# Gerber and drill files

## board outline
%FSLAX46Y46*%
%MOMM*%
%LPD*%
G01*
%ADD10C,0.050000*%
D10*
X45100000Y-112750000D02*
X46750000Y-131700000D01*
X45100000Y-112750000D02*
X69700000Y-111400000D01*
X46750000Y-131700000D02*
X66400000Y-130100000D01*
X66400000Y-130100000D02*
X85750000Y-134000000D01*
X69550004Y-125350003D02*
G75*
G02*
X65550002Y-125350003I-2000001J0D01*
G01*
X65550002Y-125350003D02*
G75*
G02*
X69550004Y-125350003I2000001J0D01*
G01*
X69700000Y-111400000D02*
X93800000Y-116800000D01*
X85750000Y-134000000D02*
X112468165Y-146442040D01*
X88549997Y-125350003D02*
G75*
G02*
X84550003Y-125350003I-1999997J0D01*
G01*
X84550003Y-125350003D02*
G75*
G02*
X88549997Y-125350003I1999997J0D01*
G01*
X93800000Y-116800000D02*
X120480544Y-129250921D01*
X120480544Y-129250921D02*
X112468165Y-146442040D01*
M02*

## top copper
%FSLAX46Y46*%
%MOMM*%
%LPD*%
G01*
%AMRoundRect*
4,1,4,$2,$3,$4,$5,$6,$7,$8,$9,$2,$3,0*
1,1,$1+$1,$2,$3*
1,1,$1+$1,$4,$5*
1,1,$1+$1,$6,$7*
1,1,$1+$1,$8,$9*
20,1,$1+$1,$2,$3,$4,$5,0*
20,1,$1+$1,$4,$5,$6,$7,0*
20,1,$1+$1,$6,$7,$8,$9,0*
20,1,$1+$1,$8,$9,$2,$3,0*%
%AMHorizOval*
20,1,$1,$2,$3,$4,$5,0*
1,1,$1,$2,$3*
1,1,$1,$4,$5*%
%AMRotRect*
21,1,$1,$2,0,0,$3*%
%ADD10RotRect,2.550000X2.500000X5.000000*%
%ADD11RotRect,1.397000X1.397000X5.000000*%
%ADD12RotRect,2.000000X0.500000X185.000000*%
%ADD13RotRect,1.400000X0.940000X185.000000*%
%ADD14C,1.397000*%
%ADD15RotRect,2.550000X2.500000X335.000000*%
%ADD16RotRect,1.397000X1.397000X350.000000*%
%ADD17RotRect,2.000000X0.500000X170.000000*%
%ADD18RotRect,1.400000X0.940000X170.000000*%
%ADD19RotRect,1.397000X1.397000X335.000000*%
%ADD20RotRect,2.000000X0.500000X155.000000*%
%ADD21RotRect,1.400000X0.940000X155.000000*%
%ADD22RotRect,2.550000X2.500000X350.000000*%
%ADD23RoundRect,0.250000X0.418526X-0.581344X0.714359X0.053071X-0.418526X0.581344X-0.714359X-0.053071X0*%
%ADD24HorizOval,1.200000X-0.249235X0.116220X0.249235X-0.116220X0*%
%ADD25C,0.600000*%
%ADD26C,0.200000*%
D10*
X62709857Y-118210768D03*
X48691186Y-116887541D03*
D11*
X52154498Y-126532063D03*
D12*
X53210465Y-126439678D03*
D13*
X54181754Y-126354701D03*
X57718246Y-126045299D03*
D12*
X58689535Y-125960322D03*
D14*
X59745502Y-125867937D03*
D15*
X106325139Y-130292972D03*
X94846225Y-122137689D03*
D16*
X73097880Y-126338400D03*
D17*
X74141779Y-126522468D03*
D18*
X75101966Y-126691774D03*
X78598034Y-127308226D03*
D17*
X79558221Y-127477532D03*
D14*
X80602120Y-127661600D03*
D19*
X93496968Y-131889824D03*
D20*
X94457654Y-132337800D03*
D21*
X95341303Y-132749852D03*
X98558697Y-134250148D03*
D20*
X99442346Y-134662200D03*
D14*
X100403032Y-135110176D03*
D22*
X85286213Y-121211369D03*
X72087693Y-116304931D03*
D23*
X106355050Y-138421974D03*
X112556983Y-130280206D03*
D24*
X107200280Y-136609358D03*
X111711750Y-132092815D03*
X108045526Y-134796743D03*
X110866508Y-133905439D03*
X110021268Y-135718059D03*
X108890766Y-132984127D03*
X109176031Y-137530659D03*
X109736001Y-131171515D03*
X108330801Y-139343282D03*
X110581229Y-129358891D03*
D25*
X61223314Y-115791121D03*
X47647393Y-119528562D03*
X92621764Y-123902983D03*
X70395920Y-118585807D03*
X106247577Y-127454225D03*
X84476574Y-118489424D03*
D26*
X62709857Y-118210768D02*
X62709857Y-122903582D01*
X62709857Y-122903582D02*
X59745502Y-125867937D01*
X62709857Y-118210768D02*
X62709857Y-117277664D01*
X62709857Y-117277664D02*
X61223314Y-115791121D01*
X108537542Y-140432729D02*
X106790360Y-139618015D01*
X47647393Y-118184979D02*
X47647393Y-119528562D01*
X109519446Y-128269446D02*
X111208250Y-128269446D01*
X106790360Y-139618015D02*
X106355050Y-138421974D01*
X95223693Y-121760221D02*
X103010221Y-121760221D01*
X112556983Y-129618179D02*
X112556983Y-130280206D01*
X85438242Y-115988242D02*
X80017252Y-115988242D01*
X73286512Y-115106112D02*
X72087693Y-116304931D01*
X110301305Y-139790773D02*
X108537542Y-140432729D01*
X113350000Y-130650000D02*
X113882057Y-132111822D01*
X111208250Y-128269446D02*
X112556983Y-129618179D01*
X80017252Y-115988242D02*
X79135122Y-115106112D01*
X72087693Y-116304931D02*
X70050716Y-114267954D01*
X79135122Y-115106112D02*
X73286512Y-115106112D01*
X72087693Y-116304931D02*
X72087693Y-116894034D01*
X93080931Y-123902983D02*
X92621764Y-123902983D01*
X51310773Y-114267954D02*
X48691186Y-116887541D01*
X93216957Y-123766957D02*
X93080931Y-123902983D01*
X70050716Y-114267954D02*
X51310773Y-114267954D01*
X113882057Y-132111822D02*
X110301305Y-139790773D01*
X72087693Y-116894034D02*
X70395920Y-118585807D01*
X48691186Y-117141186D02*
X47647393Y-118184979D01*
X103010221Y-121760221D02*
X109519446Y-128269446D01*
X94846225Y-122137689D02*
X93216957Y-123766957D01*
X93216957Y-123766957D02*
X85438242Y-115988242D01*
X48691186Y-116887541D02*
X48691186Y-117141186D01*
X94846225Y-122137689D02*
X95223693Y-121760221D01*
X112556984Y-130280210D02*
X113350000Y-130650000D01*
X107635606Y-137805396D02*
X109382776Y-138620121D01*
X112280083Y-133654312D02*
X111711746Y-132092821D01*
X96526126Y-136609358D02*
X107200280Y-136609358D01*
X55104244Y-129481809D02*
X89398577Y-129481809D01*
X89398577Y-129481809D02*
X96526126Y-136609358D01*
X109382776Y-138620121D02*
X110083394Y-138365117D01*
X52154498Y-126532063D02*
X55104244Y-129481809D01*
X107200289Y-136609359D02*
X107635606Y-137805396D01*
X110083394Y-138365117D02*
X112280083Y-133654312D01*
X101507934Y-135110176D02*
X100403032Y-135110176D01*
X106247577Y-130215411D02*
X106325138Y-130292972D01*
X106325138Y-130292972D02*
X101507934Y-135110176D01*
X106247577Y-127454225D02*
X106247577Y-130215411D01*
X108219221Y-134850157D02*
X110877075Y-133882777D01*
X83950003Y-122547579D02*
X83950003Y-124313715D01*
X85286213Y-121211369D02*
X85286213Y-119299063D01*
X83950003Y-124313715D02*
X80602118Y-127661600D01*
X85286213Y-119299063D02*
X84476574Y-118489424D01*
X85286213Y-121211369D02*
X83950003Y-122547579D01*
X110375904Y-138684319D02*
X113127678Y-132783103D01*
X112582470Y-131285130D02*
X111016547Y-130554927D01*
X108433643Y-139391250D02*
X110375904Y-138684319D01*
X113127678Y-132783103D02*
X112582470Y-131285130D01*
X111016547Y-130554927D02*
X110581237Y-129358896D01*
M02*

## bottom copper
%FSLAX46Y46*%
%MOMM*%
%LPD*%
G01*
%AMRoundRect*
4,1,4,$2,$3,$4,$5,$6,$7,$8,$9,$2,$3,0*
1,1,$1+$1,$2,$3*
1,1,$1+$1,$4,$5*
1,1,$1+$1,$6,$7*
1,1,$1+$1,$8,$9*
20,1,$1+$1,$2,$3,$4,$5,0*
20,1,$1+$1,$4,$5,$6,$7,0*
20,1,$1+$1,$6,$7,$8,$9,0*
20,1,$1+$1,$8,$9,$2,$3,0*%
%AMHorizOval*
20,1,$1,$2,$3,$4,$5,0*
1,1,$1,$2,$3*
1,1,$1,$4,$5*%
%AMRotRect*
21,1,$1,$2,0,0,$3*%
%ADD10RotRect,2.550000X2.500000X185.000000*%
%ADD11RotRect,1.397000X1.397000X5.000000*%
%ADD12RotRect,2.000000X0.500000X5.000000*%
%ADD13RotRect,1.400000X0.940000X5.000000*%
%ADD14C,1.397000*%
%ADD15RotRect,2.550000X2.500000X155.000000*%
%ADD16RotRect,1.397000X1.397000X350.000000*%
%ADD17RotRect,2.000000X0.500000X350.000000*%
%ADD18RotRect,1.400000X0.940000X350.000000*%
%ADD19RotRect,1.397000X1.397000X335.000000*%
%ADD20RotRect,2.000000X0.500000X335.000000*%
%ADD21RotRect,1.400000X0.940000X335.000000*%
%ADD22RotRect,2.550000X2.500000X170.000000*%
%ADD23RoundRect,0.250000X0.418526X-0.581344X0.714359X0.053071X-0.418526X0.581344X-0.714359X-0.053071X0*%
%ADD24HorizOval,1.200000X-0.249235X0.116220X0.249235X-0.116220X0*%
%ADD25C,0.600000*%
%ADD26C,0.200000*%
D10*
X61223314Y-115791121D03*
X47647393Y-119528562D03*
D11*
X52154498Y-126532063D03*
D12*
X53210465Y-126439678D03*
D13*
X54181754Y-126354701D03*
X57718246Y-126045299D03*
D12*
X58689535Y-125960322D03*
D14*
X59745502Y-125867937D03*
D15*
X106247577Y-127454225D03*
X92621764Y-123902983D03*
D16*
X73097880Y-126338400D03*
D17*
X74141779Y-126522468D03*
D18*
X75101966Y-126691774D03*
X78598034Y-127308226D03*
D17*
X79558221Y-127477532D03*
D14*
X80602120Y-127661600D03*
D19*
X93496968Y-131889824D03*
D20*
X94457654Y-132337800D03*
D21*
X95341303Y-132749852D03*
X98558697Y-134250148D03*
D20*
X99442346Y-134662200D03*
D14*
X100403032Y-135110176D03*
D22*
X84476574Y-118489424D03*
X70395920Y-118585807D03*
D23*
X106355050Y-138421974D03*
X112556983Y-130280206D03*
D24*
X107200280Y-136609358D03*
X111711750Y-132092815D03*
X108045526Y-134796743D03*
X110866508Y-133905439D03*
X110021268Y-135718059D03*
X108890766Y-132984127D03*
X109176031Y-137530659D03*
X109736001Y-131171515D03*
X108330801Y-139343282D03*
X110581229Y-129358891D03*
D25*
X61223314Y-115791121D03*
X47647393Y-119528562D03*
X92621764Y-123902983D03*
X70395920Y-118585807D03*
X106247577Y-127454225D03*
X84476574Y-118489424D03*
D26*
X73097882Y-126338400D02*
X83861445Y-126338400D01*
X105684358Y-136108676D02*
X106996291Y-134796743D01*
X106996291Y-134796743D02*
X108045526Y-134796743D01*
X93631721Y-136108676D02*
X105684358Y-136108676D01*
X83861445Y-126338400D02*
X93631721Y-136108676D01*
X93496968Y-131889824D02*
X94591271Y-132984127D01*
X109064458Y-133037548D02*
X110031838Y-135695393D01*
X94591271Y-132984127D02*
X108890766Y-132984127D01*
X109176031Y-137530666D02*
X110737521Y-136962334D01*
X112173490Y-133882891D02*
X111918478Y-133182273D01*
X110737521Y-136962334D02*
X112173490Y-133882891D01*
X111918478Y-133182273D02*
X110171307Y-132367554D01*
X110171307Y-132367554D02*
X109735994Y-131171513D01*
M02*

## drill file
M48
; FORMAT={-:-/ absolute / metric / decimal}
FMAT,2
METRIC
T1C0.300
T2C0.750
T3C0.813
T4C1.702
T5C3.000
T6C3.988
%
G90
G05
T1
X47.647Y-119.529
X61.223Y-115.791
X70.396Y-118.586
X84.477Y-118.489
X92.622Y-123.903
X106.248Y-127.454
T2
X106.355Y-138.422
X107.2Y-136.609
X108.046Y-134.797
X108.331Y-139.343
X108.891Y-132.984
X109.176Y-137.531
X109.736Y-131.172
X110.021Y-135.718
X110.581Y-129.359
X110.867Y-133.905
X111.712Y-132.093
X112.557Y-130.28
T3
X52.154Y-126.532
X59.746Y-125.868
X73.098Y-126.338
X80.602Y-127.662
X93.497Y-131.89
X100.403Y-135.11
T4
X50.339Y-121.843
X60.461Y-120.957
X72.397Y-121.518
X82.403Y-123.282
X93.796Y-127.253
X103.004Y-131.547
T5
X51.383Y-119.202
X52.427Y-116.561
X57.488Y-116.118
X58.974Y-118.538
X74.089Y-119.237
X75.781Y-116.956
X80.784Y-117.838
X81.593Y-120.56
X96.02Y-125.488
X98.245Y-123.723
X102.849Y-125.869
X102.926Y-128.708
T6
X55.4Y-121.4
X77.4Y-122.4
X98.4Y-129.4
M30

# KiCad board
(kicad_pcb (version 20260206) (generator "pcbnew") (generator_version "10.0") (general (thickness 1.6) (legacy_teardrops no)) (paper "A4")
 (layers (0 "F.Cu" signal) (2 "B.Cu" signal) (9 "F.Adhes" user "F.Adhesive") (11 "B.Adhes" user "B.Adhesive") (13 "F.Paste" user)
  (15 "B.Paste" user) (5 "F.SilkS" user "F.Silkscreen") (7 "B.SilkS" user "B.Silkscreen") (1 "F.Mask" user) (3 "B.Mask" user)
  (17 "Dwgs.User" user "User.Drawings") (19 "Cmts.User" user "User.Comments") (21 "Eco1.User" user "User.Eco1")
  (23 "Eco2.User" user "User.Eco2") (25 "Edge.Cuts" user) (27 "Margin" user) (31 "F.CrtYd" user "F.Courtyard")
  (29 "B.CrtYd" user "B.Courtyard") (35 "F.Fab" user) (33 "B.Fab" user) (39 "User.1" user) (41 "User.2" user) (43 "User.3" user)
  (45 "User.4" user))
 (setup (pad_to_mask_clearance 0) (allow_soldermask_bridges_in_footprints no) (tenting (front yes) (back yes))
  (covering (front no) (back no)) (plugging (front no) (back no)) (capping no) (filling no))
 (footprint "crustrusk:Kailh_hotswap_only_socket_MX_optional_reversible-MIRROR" (layer "F.Cu") (at 55.400001 121.4 5)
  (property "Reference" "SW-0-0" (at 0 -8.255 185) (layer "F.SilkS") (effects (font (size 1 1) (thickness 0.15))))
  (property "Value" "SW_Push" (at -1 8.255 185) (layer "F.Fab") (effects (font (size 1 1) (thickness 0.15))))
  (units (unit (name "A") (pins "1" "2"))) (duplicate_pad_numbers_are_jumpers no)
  (pad "" np_thru_hole circle (at -5.08 0 5) (size 1.7018 1.7018) (drill 1.7018) (layers "*.Cu" "*.Mask"))
  (pad "" np_thru_hole circle (at -3.81 -2.54 185) (size 3 3) (drill 3) (layers "*.Cu" "*.Mask"))
  (pad "" np_thru_hole circle (at -2.540002 -5.079998 5) (size 3 3) (drill 3) (layers "*.Cu" "*.Mask"))
  (pad "" np_thru_hole circle (at 0 0 5) (size 3.9878 3.9878) (drill 3.9878) (layers "*.Cu" "*.Mask"))
  (pad "" np_thru_hole circle (at 2.540002 -5.080001 185) (size 3 3) (drill 3) (layers "*.Cu" "*.Mask"))
  (pad "" np_thru_hole circle (at 3.81 -2.54 5) (size 3 3) (drill 3) (layers "*.Cu" "*.Mask"))
  (pad "" np_thru_hole circle (at 5.08 0 5) (size 1.7018 1.7018) (drill 1.7018) (layers "*.Cu" "*.Mask"))
  (pad "1" smd rect (at 6.29 -5.08 185) (size 2.55 2.5) (layers "B.Cu" "B.Mask" "B.Paste") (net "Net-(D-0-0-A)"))
  (pad "1" smd rect (at 7.56 -2.54 5) (size 2.55 2.5) (layers "F.Cu" "F.Mask" "F.Paste") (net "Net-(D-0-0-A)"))
  (pad "2" smd rect (at -7.56 -2.540001 185) (size 2.55 2.5) (layers "B.Cu" "B.Mask" "B.Paste") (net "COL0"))
  (pad "2" smd rect (at -6.289999 -5.079999 5) (size 2.55 2.5) (layers "F.Cu" "F.Mask" "F.Paste") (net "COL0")))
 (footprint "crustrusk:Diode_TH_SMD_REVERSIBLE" (layer "F.Cu") (at 55.95 126.2 5)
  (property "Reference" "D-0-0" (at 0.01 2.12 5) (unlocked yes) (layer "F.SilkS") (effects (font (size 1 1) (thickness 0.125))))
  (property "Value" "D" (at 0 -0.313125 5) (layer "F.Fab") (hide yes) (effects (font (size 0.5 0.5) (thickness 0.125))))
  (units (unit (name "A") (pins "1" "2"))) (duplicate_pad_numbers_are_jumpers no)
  (pad "1" thru_hole rect (at -3.81 0 5) (size 1.397 1.397) (drill 0.8128) (layers "*.Cu" "*.Mask") (remove_unused_layers no) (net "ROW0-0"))
  (pad "1" smd rect (at -2.75 0 185) (size 2 0.5) (layers "F.Cu") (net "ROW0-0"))
  (pad "1" smd rect (at -2.75 0 5) (size 2 0.5) (layers "B.Cu") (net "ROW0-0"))
  (pad "1" smd rect (at -1.775 0 185) (size 1.4 0.94) (layers "F.Cu" "F.Mask" "F.Paste") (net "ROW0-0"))
  (pad "1" smd rect (at -1.775 0 5) (size 1.4 0.94) (layers "B.Cu" "B.Mask" "B.Paste") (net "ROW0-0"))
  (pad "2" smd rect (at 1.775 0 185) (size 1.4 0.94) (layers "F.Cu" "F.Mask" "F.Paste") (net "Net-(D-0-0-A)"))
  (pad "2" smd rect (at 1.775 0 5) (size 1.4 0.94) (layers "B.Cu" "B.Mask" "B.Paste") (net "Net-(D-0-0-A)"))
  (pad "2" smd rect (at 2.75 0 185) (size 2 0.5) (layers "F.Cu") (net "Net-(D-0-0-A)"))
  (pad "2" smd rect (at 2.75 0 5) (size 2 0.5) (layers "B.Cu") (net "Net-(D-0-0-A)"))
  (pad "2" thru_hole circle (at 3.81 0 5) (size 1.397 1.397) (drill 0.8128) (layers "*.Cu" "*.Mask") (remove_unused_layers no)
   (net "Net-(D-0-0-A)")))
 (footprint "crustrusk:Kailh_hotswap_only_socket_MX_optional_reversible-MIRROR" (layer "F.Cu") (at 98.4 129.4 -25)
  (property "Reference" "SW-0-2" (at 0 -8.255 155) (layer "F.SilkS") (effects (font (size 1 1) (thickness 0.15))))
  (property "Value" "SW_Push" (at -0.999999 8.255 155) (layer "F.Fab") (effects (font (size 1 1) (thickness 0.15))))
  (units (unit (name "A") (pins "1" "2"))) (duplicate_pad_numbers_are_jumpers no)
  (pad "" np_thru_hole circle (at -5.08 0 335) (size 1.7018 1.7018) (drill 1.7018) (layers "*.Cu" "*.Mask"))
  (pad "" np_thru_hole circle (at -3.81 -2.539998 155) (size 3 3) (drill 3) (layers "*.Cu" "*.Mask"))
  (pad "" np_thru_hole circle (at -2.54 -5.079998 335) (size 3 3) (drill 3) (layers "*.Cu" "*.Mask"))
  (pad "" np_thru_hole circle (at 0 0 335) (size 3.9878 3.9878) (drill 3.9878) (layers "*.Cu" "*.Mask"))
  (pad "" np_thru_hole circle (at 2.540002 -5.080001 155) (size 3 3) (drill 3) (layers "*.Cu" "*.Mask"))
  (pad "" np_thru_hole circle (at 3.81 -2.54 335) (size 3 3) (drill 3) (layers "*.Cu" "*.Mask"))
  (pad "" np_thru_hole circle (at 5.08 0 335) (size 1.7018 1.7018) (drill 1.7018) (layers "*.Cu" "*.Mask"))
  (pad "1" smd rect (at 6.29 -5.08 155) (size 2.55 2.5) (layers "B.Cu" "B.Mask" "B.Paste") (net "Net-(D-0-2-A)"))
  (pad "1" smd rect (at 7.560001 -2.540001 335) (size 2.55 2.5) (layers "F.Cu" "F.Mask" "F.Paste") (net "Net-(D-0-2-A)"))
  (pad "2" smd rect (at -7.56 -2.540001 155) (size 2.55 2.5) (layers "B.Cu" "B.Mask" "B.Paste") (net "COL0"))
  (pad "2" smd rect (at -6.289999 -5.079999 335) (size 2.55 2.5) (layers "F.Cu" "F.Mask" "F.Paste") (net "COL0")))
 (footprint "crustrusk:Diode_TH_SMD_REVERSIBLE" (layer "F.Cu") (at 76.85 127 -10)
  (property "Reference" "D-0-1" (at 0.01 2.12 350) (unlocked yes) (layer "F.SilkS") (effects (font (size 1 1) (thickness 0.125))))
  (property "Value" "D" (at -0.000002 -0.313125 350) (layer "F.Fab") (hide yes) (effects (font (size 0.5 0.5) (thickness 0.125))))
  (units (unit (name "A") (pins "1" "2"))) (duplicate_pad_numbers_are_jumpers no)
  (pad "1" thru_hole rect (at -3.810002 0 350) (size 1.397 1.397) (drill 0.8128) (layers "*.Cu" "*.Mask") (remove_unused_layers no)
   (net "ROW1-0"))
  (pad "1" smd rect (at -2.75 0 170) (size 2 0.5) (layers "F.Cu") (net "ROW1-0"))
  (pad "1" smd rect (at -2.75 0 350) (size 2 0.5) (layers "B.Cu") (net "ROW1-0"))
  (pad "1" smd rect (at -1.775 0 170) (size 1.4 0.94) (layers "F.Cu" "F.Mask" "F.Paste") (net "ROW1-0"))
  (pad "1" smd rect (at -1.775 0 350) (size 1.4 0.94) (layers "B.Cu" "B.Mask" "B.Paste") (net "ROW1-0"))
  (pad "2" smd rect (at 1.775 0 170) (size 1.4 0.94) (layers "F.Cu" "F.Mask" "F.Paste") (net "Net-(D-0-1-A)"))
  (pad "2" smd rect (at 1.775 0 350) (size 1.4 0.94) (layers "B.Cu" "B.Mask" "B.Paste") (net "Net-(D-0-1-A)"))
  (pad "2" smd rect (at 2.75 0 170) (size 2 0.5) (layers "F.Cu") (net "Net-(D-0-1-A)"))
  (pad "2" smd rect (at 2.75 0 350) (size 2 0.5) (layers "B.Cu") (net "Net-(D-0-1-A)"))
  (pad "2" thru_hole circle (at 3.810002 0 350) (size 1.397 1.397) (drill 0.8128) (layers "*.Cu" "*.Mask") (remove_unused_layers no)
   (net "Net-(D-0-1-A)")))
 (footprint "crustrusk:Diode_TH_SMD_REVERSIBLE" (layer "F.Cu") (at 96.95 133.5 -25)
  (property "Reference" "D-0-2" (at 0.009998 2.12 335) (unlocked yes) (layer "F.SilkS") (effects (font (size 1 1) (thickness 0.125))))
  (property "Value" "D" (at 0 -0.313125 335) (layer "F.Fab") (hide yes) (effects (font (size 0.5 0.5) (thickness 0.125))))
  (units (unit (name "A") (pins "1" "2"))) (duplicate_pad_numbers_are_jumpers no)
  (pad "1" thru_hole rect (at -3.81 -0.000001 335) (size 1.397 1.397) (drill 0.8128) (layers "*.Cu" "*.Mask") (remove_unused_layers no)
   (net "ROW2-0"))
  (pad "1" smd rect (at -2.75 0 155) (size 2 0.5) (layers "F.Cu") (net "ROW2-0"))
  (pad "1" smd rect (at -2.75 0 335) (size 2 0.5) (layers "B.Cu") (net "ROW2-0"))
  (pad "1" smd rect (at -1.775001 0 155) (size 1.4 0.94) (layers "F.Cu" "F.Mask" "F.Paste") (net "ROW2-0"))
  (pad "1" smd rect (at -1.775001 0 335) (size 1.4 0.94) (layers "B.Cu" "B.Mask" "B.Paste") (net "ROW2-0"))
  (pad "2" smd rect (at 1.775001 0 155) (size 1.4 0.94) (layers "F.Cu" "F.Mask" "F.Paste") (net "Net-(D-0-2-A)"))
  (pad "2" smd rect (at 1.775001 0 335) (size 1.4 0.94) (layers "B.Cu" "B.Mask" "B.Paste") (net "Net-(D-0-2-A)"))
  (pad "2" smd rect (at 2.75 0 155) (size 2 0.5) (layers "F.Cu") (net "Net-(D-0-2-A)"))
  (pad "2" smd rect (at 2.75 0 335) (size 2 0.5) (layers "B.Cu") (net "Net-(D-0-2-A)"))
  (pad "2" thru_hole circle (at 3.81 0.000001 335) (size 1.397 1.397) (drill 0.8128) (layers "*.Cu" "*.Mask") (remove_unused_layers no)
   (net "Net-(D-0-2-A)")))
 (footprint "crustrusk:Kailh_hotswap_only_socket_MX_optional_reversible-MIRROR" (layer "F.Cu") (at 77.4 122.4 -10)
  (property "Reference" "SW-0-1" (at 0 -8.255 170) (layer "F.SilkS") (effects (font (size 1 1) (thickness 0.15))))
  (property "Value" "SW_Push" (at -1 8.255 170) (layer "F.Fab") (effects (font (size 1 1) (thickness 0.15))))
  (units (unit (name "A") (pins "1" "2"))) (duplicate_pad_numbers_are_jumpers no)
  (pad "" np_thru_hole circle (at -5.08 0 350) (size 1.7018 1.7018) (drill 1.7018) (layers "*.Cu" "*.Mask"))
  (pad "" np_thru_hole circle (at -3.81 -2.54 170) (size 3 3) (drill 3) (layers "*.Cu" "*.Mask"))
  (pad "" np_thru_hole circle (at -2.54 -5.079998 350) (size 3 3) (drill 3) (layers "*.Cu" "*.Mask"))
  (pad "" np_thru_hole circle (at 0 0 350) (size 3.9878 3.9878) (drill 3.9878) (layers "*.Cu" "*.Mask"))
  (pad "" np_thru_hole circle (at 2.540002 -5.080001 170) (size 3 3) (drill 3) (layers "*.Cu" "*.Mask"))
  (pad "" np_thru_hole circle (at 3.81 -2.54 350) (size 3 3) (drill 3) (layers "*.Cu" "*.Mask"))
  (pad "" np_thru_hole circle (at 5.08 0 350) (size 1.7018 1.7018) (drill 1.7018) (layers "*.Cu" "*.Mask"))
  (pad "1" smd rect (at 6.290001 -5.08 170) (size 2.55 2.5) (layers "B.Cu" "B.Mask" "B.Paste") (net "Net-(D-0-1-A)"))
  (pad "1" smd rect (at 7.56 -2.54 350) (size 2.55 2.5) (layers "F.Cu" "F.Mask" "F.Paste") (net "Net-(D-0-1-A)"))
  (pad "2" smd rect (at -7.56 -2.540001 170) (size 2.55 2.5) (layers "B.Cu" "B.Mask" "B.Paste") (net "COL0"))
  (pad "2" smd rect (at -6.289999 -5.079999 350) (size 2.55 2.5) (layers "F.Cu" "F.Mask" "F.Paste") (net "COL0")))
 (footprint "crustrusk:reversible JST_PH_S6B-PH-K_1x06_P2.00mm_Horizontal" (layer "F.Cu") (at 106.35505 138.421974 65)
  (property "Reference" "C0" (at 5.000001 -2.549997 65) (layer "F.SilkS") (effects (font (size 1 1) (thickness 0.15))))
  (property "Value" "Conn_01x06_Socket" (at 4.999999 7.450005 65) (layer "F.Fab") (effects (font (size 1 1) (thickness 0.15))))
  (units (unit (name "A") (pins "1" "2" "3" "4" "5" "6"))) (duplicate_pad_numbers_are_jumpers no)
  (pad "1" thru_hole roundrect (at 0 0 65) (size 1.2 1.75) (drill 0.75) (layers "*.Cu" "*.Mask") (remove_unused_layers no)
   (roundrect_rratio 0.208333) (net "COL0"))
  (pad "1" thru_hole roundrect (at 9.999998 2.18 65) (size 1.2 1.75) (drill 0.75) (layers "*.Cu" "*.Mask") (remove_unused_layers no)
   (roundrect_rratio 0.208333) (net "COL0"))
  (pad "2" thru_hole oval (at 1.999998 -0.000006 65) (size 1.2 1.75) (drill 0.75) (layers "*.Cu" "*.Mask") (remove_unused_layers no)
   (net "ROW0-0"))
  (pad "2" thru_hole oval (at 8.000005 2.180001 65) (size 1.2 1.75) (drill 0.75) (layers "*.Cu" "*.Mask") (remove_unused_layers no)
   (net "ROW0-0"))
  (pad "3" thru_hole oval (at 4.000001 0.000003 65) (size 1.2 1.75) (drill 0.75) (layers "*.Cu" "*.Mask") (remove_unused_layers no)
   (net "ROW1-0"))
  (pad "3" thru_hole oval (at 5.999995 2.179999 65) (size 1.2 1.75) (drill 0.75) (layers "*.Cu" "*.Mask") (remove_unused_layers no)
   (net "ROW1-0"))
  (pad "4" thru_hole oval (at 3.99999 2.179998 65) (size 1.2 1.75) (drill 0.75) (layers "*.Cu" "*.Mask") (remove_unused_layers no)
   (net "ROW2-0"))
  (pad "4" thru_hole oval (at 6.000003 0.000006 65) (size 1.2 1.75) (drill 0.75) (layers "*.Cu" "*.Mask") (remove_unused_layers no)
   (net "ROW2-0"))
  (pad "5" thru_hole oval (at 2.000004 2.179991 65) (size 1.2 1.75) (drill 0.75) (layers "*.Cu" "*.Mask") (remove_unused_layers no)
   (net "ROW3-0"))
  (pad "5" thru_hole oval (at 7.999999 0.000006 65) (size 1.2 1.75) (drill 0.75) (layers "*.Cu" "*.Mask") (remove_unused_layers no)
   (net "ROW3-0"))
  (pad "6" thru_hole oval (at 0 2.18 65) (size 1.2 1.75) (drill 0.75) (layers "*.Cu" "*.Mask") (remove_unused_layers no) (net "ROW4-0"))
  (pad "6" thru_hole oval (at 10.000003 -0.000005 65) (size 1.2 1.75) (drill 0.75) (layers "*.Cu" "*.Mask") (remove_unused_layers no)
   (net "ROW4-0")))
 (gr_line (start 45.1 112.75) (end 46.75 131.7) (stroke (width 0.05) (type default)) (layer "Edge.Cuts"))
 (gr_line (start 45.1 112.75) (end 69.7 111.4) (stroke (width 0.05) (type default)) (layer "Edge.Cuts"))
 (gr_line (start 46.75 131.7) (end 66.4 130.1) (stroke (width 0.05) (type default)) (layer "Edge.Cuts"))
 (gr_line (start 66.4 130.1) (end 85.75 134) (stroke (width 0.05) (type default)) (layer "Edge.Cuts"))
 (gr_circle (center 67.550003 125.350003) (end 65.550002 125.350003) (stroke (width 0.05) (type default)) (fill no) (layer "Edge.Cuts"))
 (gr_line (start 69.7 111.4) (end 93.8 116.8) (stroke (width 0.05) (type default)) (layer "Edge.Cuts"))
 (gr_line (start 85.75 134) (end 112.468165 146.44204) (stroke (width 0.05) (type default)) (layer "Edge.Cuts"))
 (gr_circle (center 86.55 125.350003) (end 84.550003 125.350003) (stroke (width 0.05) (type default)) (fill no) (layer "Edge.Cuts"))
 (gr_line (start 93.8 116.8) (end 120.480544 129.250921) (stroke (width 0.05) (type default)) (layer "Edge.Cuts"))
 (gr_line (start 120.480544 129.250921) (end 112.468165 146.44204) (stroke (width 0.05) (type default)) (layer "Edge.Cuts"))
 (segment (start 62.709857 118.210768) (end 62.709857 122.903582) (width 0.2) (layer "F.Cu") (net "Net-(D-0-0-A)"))
 (segment (start 62.709857 122.903582) (end 59.745502 125.867937) (width 0.2) (layer "F.Cu") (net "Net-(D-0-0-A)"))
 (segment (start 62.709857 118.210768) (end 62.709857 117.277664) (width 0.2) (layer "F.Cu") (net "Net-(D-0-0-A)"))
 (segment (start 62.709857 117.277664) (end 61.223314 115.791121) (width 0.2) (layer "F.Cu") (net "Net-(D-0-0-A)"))
 (via (at 61.223314 115.791121) (size 0.6) (drill 0.3) (layers "F.Cu" "B.Cu") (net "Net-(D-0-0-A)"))
 (segment (start 108.537542 140.432729) (end 106.79036 139.618015) (width 0.2) (layer "F.Cu") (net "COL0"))
 (segment (start 47.647393 118.184979) (end 47.647393 119.528562) (width 0.2) (layer "F.Cu") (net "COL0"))
 (segment (start 109.519446 128.269446) (end 111.20825 128.269446) (width 0.2) (layer "F.Cu") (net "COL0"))
 (segment (start 106.79036 139.618015) (end 106.35505 138.421974) (width 0.2) (layer "F.Cu") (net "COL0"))
 (segment (start 95.223693 121.760221) (end 103.010221 121.760221) (width 0.2) (layer "F.Cu") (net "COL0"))
 (segment (start 112.556983 129.618179) (end 112.556983 130.280206) (width 0.2) (layer "F.Cu") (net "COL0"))
 (segment (start 85.438242 115.988242) (end 80.017252 115.988242) (width 0.2) (layer "F.Cu") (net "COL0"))
 (segment (start 73.286512 115.106112) (end 72.087693 116.304931) (width 0.2) (layer "F.Cu") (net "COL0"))
 (segment (start 110.301305 139.790773) (end 108.537542 140.432729) (width 0.2) (layer "F.Cu") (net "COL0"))
 (segment (start 113.35 130.65) (end 113.882057 132.111822) (width 0.2) (layer "F.Cu") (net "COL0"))
 (segment (start 111.20825 128.269446) (end 112.556983 129.618179) (width 0.2) (layer "F.Cu") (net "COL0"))
 (segment (start 80.017252 115.988242) (end 79.135122 115.106112) (width 0.2) (layer "F.Cu") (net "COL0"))
 (segment (start 72.087693 116.304931) (end 70.050716 114.267954) (width 0.2) (layer "F.Cu") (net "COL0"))
 (segment (start 79.135122 115.106112) (end 73.286512 115.106112) (width 0.2) (layer "F.Cu") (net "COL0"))
 (segment (start 72.087693 116.304931) (end 72.087693 116.894034) (width 0.2) (layer "F.Cu") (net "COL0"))
 (segment (start 93.080931 123.902983) (end 92.621764 123.902983) (width 0.2) (layer "F.Cu") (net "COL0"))
 (segment (start 51.310773 114.267954) (end 48.691186 116.887541) (width 0.2) (layer "F.Cu") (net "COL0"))
 (segment (start 93.216957 123.766957) (end 93.080931 123.902983) (width 0.2) (layer "F.Cu") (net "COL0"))
 (segment (start 70.050716 114.267954) (end 51.310773 114.267954) (width 0.2) (layer "F.Cu") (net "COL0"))
 (segment (start 113.882057 132.111822) (end 110.301305 139.790773) (width 0.2) (layer "F.Cu") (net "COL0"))
 (segment (start 72.087693 116.894034) (end 70.39592 118.585807) (width 0.2) (layer "F.Cu") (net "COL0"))
 (segment (start 48.691186 117.141186) (end 47.647393 118.184979) (width 0.2) (layer "F.Cu") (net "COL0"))
 (segment (start 103.010221 121.760221) (end 109.519446 128.269446) (width 0.2) (layer "F.Cu") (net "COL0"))
 (segment (start 94.846225 122.137689) (end 93.216957 123.766957) (width 0.2) (layer "F.Cu") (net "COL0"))
 (segment (start 93.216957 123.766957) (end 85.438242 115.988242) (width 0.2) (layer "F.Cu") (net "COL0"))
 (segment (start 48.691186 116.887541) (end 48.691186 117.141186) (width 0.2) (layer "F.Cu") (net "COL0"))
 (segment (start 94.846225 122.137689) (end 95.223693 121.760221) (width 0.2) (layer "F.Cu") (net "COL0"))
 (segment (start 112.556984 130.28021) (end 113.35 130.65) (width 0.2) (layer "F.Cu") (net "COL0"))
 (via (at 47.647393 119.528562) (size 0.6) (drill 0.3) (layers "F.Cu" "B.Cu") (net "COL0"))
 (via (at 92.621764 123.902983) (size 0.6) (drill 0.3) (layers "F.Cu" "B.Cu") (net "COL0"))
 (via (at 70.39592 118.585807) (size 0.6) (drill 0.3) (layers "F.Cu" "B.Cu") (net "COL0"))
 (segment (start 107.635606 137.805396) (end 109.382776 138.620121) (width 0.2) (layer "F.Cu") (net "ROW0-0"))
 (segment (start 112.280083 133.654312) (end 111.711746 132.092821) (width 0.2) (layer "F.Cu") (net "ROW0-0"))
 (segment (start 96.526126 136.609358) (end 107.20028 136.609358) (width 0.2) (layer "F.Cu") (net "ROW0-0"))
 (segment (start 55.104244 129.481809) (end 89.398577 129.481809) (width 0.2) (layer "F.Cu") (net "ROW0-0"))
 (segment (start 89.398577 129.481809) (end 96.526126 136.609358) (width 0.2) (layer "F.Cu") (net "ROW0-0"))
 (segment (start 109.382776 138.620121) (end 110.083394 138.365117) (width 0.2) (layer "F.Cu") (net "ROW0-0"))
 (segment (start 52.154498 126.532063) (end 55.104244 129.481809) (width 0.2) (layer "F.Cu") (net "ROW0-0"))
 (segment (start 107.200289 136.609359) (end 107.635606 137.805396) (width 0.2) (layer "F.Cu") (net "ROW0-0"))
 (segment (start 110.083394 138.365117) (end 112.280083 133.654312) (width 0.2) (layer "F.Cu") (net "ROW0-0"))
 (segment (start 101.507934 135.110176) (end 100.403032 135.110176) (width 0.2) (layer "F.Cu") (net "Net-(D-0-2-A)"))
 (segment (start 106.247577 130.215411) (end 106.325138 130.292972) (width 0.2) (layer "F.Cu") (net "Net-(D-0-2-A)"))
 (segment (start 106.325138 130.292972) (end 101.507934 135.110176) (width 0.2) (layer "F.Cu") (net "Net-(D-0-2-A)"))
 (segment (start 106.247577 127.454225) (end 106.247577 130.215411) (width 0.2) (layer "F.Cu") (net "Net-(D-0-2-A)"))
 (via (at 106.247577 127.454225) (size 0.6) (drill 0.3) (layers "F.Cu" "B.Cu") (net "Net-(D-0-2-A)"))
 (segment (start 108.219221 134.850157) (end 110.877075 133.882777) (width 0.2) (layer "F.Cu") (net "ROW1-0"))
 (segment (start 73.097882 126.3384) (end 83.861445 126.3384) (width 0.2) (layer "B.Cu") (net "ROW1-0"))
 (segment (start 105.684358 136.108676) (end 106.996291 134.796743) (width 0.2) (layer "B.Cu") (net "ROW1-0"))
 (segment (start 106.996291 134.796743) (end 108.045526 134.796743) (width 0.2) (layer "B.Cu") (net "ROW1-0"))
 (segment (start 93.631721 136.108676) (end 105.684358 136.108676) (width 0.2) (layer "B.Cu") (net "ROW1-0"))
 (segment (start 83.861445 126.3384) (end 93.631721 136.108676) (width 0.2) (layer "B.Cu") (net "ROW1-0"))
 (segment (start 83.950003 122.547579) (end 83.950003 124.313715) (width 0.2) (layer "F.Cu") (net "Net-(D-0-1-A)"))
 (segment (start 85.286213 121.211369) (end 85.286213 119.299063) (width 0.2) (layer "F.Cu") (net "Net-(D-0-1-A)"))
 (segment (start 83.950003 124.313715) (end 80.602118 127.6616) (width 0.2) (layer "F.Cu") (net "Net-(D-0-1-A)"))
 (segment (start 85.286213 119.299063) (end 84.476574 118.489424) (width 0.2) (layer "F.Cu") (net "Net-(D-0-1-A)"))
 (segment (start 85.286213 121.211369) (end 83.950003 122.547579) (width 0.2) (layer "F.Cu") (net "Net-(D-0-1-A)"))
 (via (at 84.476574 118.489424) (size 0.6) (drill 0.3) (layers "F.Cu" "B.Cu") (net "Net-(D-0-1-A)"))
 (segment (start 93.496968 131.889824) (end 94.591271 132.984127) (width 0.2) (layer "B.Cu") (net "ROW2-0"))
 (segment (start 109.064458 133.037548) (end 110.031838 135.695393) (width 0.2) (layer "B.Cu") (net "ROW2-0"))
 (segment (start 94.591271 132.984127) (end 108.890766 132.984127) (width 0.2) (layer "B.Cu") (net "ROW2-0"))
 (segment (start 109.176031 137.530666) (end 110.737521 136.962334) (width 0.2) (layer "B.Cu") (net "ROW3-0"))
 (segment (start 112.17349 133.882891) (end 111.918478 133.182273) (width 0.2) (layer "B.Cu") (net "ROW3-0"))
 (segment (start 110.737521 136.962334) (end 112.17349 133.882891) (width 0.2) (layer "B.Cu") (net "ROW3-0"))
 (segment (start 111.918478 133.182273) (end 110.171307 132.367554) (width 0.2) (layer "B.Cu") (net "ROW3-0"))
 (segment (start 110.171307 132.367554) (end 109.735994 131.171513) (width 0.2) (layer "B.Cu") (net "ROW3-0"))
 (segment (start 110.375904 138.684319) (end 113.127678 132.783103) (width 0.2) (layer "F.Cu") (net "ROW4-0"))
 (segment (start 112.58247 131.28513) (end 111.016547 130.554927) (width 0.2) (layer "F.Cu") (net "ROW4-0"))
 (segment (start 108.433643 139.39125) (end 110.375904 138.684319) (width 0.2) (layer "F.Cu") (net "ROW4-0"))
 (segment (start 113.127678 132.783103) (end 112.58247 131.28513) (width 0.2) (layer "F.Cu") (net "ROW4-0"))
 (segment (start 111.016547 130.554927) (end 110.581237 129.358896) (width 0.2) (layer "F.Cu") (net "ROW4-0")))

